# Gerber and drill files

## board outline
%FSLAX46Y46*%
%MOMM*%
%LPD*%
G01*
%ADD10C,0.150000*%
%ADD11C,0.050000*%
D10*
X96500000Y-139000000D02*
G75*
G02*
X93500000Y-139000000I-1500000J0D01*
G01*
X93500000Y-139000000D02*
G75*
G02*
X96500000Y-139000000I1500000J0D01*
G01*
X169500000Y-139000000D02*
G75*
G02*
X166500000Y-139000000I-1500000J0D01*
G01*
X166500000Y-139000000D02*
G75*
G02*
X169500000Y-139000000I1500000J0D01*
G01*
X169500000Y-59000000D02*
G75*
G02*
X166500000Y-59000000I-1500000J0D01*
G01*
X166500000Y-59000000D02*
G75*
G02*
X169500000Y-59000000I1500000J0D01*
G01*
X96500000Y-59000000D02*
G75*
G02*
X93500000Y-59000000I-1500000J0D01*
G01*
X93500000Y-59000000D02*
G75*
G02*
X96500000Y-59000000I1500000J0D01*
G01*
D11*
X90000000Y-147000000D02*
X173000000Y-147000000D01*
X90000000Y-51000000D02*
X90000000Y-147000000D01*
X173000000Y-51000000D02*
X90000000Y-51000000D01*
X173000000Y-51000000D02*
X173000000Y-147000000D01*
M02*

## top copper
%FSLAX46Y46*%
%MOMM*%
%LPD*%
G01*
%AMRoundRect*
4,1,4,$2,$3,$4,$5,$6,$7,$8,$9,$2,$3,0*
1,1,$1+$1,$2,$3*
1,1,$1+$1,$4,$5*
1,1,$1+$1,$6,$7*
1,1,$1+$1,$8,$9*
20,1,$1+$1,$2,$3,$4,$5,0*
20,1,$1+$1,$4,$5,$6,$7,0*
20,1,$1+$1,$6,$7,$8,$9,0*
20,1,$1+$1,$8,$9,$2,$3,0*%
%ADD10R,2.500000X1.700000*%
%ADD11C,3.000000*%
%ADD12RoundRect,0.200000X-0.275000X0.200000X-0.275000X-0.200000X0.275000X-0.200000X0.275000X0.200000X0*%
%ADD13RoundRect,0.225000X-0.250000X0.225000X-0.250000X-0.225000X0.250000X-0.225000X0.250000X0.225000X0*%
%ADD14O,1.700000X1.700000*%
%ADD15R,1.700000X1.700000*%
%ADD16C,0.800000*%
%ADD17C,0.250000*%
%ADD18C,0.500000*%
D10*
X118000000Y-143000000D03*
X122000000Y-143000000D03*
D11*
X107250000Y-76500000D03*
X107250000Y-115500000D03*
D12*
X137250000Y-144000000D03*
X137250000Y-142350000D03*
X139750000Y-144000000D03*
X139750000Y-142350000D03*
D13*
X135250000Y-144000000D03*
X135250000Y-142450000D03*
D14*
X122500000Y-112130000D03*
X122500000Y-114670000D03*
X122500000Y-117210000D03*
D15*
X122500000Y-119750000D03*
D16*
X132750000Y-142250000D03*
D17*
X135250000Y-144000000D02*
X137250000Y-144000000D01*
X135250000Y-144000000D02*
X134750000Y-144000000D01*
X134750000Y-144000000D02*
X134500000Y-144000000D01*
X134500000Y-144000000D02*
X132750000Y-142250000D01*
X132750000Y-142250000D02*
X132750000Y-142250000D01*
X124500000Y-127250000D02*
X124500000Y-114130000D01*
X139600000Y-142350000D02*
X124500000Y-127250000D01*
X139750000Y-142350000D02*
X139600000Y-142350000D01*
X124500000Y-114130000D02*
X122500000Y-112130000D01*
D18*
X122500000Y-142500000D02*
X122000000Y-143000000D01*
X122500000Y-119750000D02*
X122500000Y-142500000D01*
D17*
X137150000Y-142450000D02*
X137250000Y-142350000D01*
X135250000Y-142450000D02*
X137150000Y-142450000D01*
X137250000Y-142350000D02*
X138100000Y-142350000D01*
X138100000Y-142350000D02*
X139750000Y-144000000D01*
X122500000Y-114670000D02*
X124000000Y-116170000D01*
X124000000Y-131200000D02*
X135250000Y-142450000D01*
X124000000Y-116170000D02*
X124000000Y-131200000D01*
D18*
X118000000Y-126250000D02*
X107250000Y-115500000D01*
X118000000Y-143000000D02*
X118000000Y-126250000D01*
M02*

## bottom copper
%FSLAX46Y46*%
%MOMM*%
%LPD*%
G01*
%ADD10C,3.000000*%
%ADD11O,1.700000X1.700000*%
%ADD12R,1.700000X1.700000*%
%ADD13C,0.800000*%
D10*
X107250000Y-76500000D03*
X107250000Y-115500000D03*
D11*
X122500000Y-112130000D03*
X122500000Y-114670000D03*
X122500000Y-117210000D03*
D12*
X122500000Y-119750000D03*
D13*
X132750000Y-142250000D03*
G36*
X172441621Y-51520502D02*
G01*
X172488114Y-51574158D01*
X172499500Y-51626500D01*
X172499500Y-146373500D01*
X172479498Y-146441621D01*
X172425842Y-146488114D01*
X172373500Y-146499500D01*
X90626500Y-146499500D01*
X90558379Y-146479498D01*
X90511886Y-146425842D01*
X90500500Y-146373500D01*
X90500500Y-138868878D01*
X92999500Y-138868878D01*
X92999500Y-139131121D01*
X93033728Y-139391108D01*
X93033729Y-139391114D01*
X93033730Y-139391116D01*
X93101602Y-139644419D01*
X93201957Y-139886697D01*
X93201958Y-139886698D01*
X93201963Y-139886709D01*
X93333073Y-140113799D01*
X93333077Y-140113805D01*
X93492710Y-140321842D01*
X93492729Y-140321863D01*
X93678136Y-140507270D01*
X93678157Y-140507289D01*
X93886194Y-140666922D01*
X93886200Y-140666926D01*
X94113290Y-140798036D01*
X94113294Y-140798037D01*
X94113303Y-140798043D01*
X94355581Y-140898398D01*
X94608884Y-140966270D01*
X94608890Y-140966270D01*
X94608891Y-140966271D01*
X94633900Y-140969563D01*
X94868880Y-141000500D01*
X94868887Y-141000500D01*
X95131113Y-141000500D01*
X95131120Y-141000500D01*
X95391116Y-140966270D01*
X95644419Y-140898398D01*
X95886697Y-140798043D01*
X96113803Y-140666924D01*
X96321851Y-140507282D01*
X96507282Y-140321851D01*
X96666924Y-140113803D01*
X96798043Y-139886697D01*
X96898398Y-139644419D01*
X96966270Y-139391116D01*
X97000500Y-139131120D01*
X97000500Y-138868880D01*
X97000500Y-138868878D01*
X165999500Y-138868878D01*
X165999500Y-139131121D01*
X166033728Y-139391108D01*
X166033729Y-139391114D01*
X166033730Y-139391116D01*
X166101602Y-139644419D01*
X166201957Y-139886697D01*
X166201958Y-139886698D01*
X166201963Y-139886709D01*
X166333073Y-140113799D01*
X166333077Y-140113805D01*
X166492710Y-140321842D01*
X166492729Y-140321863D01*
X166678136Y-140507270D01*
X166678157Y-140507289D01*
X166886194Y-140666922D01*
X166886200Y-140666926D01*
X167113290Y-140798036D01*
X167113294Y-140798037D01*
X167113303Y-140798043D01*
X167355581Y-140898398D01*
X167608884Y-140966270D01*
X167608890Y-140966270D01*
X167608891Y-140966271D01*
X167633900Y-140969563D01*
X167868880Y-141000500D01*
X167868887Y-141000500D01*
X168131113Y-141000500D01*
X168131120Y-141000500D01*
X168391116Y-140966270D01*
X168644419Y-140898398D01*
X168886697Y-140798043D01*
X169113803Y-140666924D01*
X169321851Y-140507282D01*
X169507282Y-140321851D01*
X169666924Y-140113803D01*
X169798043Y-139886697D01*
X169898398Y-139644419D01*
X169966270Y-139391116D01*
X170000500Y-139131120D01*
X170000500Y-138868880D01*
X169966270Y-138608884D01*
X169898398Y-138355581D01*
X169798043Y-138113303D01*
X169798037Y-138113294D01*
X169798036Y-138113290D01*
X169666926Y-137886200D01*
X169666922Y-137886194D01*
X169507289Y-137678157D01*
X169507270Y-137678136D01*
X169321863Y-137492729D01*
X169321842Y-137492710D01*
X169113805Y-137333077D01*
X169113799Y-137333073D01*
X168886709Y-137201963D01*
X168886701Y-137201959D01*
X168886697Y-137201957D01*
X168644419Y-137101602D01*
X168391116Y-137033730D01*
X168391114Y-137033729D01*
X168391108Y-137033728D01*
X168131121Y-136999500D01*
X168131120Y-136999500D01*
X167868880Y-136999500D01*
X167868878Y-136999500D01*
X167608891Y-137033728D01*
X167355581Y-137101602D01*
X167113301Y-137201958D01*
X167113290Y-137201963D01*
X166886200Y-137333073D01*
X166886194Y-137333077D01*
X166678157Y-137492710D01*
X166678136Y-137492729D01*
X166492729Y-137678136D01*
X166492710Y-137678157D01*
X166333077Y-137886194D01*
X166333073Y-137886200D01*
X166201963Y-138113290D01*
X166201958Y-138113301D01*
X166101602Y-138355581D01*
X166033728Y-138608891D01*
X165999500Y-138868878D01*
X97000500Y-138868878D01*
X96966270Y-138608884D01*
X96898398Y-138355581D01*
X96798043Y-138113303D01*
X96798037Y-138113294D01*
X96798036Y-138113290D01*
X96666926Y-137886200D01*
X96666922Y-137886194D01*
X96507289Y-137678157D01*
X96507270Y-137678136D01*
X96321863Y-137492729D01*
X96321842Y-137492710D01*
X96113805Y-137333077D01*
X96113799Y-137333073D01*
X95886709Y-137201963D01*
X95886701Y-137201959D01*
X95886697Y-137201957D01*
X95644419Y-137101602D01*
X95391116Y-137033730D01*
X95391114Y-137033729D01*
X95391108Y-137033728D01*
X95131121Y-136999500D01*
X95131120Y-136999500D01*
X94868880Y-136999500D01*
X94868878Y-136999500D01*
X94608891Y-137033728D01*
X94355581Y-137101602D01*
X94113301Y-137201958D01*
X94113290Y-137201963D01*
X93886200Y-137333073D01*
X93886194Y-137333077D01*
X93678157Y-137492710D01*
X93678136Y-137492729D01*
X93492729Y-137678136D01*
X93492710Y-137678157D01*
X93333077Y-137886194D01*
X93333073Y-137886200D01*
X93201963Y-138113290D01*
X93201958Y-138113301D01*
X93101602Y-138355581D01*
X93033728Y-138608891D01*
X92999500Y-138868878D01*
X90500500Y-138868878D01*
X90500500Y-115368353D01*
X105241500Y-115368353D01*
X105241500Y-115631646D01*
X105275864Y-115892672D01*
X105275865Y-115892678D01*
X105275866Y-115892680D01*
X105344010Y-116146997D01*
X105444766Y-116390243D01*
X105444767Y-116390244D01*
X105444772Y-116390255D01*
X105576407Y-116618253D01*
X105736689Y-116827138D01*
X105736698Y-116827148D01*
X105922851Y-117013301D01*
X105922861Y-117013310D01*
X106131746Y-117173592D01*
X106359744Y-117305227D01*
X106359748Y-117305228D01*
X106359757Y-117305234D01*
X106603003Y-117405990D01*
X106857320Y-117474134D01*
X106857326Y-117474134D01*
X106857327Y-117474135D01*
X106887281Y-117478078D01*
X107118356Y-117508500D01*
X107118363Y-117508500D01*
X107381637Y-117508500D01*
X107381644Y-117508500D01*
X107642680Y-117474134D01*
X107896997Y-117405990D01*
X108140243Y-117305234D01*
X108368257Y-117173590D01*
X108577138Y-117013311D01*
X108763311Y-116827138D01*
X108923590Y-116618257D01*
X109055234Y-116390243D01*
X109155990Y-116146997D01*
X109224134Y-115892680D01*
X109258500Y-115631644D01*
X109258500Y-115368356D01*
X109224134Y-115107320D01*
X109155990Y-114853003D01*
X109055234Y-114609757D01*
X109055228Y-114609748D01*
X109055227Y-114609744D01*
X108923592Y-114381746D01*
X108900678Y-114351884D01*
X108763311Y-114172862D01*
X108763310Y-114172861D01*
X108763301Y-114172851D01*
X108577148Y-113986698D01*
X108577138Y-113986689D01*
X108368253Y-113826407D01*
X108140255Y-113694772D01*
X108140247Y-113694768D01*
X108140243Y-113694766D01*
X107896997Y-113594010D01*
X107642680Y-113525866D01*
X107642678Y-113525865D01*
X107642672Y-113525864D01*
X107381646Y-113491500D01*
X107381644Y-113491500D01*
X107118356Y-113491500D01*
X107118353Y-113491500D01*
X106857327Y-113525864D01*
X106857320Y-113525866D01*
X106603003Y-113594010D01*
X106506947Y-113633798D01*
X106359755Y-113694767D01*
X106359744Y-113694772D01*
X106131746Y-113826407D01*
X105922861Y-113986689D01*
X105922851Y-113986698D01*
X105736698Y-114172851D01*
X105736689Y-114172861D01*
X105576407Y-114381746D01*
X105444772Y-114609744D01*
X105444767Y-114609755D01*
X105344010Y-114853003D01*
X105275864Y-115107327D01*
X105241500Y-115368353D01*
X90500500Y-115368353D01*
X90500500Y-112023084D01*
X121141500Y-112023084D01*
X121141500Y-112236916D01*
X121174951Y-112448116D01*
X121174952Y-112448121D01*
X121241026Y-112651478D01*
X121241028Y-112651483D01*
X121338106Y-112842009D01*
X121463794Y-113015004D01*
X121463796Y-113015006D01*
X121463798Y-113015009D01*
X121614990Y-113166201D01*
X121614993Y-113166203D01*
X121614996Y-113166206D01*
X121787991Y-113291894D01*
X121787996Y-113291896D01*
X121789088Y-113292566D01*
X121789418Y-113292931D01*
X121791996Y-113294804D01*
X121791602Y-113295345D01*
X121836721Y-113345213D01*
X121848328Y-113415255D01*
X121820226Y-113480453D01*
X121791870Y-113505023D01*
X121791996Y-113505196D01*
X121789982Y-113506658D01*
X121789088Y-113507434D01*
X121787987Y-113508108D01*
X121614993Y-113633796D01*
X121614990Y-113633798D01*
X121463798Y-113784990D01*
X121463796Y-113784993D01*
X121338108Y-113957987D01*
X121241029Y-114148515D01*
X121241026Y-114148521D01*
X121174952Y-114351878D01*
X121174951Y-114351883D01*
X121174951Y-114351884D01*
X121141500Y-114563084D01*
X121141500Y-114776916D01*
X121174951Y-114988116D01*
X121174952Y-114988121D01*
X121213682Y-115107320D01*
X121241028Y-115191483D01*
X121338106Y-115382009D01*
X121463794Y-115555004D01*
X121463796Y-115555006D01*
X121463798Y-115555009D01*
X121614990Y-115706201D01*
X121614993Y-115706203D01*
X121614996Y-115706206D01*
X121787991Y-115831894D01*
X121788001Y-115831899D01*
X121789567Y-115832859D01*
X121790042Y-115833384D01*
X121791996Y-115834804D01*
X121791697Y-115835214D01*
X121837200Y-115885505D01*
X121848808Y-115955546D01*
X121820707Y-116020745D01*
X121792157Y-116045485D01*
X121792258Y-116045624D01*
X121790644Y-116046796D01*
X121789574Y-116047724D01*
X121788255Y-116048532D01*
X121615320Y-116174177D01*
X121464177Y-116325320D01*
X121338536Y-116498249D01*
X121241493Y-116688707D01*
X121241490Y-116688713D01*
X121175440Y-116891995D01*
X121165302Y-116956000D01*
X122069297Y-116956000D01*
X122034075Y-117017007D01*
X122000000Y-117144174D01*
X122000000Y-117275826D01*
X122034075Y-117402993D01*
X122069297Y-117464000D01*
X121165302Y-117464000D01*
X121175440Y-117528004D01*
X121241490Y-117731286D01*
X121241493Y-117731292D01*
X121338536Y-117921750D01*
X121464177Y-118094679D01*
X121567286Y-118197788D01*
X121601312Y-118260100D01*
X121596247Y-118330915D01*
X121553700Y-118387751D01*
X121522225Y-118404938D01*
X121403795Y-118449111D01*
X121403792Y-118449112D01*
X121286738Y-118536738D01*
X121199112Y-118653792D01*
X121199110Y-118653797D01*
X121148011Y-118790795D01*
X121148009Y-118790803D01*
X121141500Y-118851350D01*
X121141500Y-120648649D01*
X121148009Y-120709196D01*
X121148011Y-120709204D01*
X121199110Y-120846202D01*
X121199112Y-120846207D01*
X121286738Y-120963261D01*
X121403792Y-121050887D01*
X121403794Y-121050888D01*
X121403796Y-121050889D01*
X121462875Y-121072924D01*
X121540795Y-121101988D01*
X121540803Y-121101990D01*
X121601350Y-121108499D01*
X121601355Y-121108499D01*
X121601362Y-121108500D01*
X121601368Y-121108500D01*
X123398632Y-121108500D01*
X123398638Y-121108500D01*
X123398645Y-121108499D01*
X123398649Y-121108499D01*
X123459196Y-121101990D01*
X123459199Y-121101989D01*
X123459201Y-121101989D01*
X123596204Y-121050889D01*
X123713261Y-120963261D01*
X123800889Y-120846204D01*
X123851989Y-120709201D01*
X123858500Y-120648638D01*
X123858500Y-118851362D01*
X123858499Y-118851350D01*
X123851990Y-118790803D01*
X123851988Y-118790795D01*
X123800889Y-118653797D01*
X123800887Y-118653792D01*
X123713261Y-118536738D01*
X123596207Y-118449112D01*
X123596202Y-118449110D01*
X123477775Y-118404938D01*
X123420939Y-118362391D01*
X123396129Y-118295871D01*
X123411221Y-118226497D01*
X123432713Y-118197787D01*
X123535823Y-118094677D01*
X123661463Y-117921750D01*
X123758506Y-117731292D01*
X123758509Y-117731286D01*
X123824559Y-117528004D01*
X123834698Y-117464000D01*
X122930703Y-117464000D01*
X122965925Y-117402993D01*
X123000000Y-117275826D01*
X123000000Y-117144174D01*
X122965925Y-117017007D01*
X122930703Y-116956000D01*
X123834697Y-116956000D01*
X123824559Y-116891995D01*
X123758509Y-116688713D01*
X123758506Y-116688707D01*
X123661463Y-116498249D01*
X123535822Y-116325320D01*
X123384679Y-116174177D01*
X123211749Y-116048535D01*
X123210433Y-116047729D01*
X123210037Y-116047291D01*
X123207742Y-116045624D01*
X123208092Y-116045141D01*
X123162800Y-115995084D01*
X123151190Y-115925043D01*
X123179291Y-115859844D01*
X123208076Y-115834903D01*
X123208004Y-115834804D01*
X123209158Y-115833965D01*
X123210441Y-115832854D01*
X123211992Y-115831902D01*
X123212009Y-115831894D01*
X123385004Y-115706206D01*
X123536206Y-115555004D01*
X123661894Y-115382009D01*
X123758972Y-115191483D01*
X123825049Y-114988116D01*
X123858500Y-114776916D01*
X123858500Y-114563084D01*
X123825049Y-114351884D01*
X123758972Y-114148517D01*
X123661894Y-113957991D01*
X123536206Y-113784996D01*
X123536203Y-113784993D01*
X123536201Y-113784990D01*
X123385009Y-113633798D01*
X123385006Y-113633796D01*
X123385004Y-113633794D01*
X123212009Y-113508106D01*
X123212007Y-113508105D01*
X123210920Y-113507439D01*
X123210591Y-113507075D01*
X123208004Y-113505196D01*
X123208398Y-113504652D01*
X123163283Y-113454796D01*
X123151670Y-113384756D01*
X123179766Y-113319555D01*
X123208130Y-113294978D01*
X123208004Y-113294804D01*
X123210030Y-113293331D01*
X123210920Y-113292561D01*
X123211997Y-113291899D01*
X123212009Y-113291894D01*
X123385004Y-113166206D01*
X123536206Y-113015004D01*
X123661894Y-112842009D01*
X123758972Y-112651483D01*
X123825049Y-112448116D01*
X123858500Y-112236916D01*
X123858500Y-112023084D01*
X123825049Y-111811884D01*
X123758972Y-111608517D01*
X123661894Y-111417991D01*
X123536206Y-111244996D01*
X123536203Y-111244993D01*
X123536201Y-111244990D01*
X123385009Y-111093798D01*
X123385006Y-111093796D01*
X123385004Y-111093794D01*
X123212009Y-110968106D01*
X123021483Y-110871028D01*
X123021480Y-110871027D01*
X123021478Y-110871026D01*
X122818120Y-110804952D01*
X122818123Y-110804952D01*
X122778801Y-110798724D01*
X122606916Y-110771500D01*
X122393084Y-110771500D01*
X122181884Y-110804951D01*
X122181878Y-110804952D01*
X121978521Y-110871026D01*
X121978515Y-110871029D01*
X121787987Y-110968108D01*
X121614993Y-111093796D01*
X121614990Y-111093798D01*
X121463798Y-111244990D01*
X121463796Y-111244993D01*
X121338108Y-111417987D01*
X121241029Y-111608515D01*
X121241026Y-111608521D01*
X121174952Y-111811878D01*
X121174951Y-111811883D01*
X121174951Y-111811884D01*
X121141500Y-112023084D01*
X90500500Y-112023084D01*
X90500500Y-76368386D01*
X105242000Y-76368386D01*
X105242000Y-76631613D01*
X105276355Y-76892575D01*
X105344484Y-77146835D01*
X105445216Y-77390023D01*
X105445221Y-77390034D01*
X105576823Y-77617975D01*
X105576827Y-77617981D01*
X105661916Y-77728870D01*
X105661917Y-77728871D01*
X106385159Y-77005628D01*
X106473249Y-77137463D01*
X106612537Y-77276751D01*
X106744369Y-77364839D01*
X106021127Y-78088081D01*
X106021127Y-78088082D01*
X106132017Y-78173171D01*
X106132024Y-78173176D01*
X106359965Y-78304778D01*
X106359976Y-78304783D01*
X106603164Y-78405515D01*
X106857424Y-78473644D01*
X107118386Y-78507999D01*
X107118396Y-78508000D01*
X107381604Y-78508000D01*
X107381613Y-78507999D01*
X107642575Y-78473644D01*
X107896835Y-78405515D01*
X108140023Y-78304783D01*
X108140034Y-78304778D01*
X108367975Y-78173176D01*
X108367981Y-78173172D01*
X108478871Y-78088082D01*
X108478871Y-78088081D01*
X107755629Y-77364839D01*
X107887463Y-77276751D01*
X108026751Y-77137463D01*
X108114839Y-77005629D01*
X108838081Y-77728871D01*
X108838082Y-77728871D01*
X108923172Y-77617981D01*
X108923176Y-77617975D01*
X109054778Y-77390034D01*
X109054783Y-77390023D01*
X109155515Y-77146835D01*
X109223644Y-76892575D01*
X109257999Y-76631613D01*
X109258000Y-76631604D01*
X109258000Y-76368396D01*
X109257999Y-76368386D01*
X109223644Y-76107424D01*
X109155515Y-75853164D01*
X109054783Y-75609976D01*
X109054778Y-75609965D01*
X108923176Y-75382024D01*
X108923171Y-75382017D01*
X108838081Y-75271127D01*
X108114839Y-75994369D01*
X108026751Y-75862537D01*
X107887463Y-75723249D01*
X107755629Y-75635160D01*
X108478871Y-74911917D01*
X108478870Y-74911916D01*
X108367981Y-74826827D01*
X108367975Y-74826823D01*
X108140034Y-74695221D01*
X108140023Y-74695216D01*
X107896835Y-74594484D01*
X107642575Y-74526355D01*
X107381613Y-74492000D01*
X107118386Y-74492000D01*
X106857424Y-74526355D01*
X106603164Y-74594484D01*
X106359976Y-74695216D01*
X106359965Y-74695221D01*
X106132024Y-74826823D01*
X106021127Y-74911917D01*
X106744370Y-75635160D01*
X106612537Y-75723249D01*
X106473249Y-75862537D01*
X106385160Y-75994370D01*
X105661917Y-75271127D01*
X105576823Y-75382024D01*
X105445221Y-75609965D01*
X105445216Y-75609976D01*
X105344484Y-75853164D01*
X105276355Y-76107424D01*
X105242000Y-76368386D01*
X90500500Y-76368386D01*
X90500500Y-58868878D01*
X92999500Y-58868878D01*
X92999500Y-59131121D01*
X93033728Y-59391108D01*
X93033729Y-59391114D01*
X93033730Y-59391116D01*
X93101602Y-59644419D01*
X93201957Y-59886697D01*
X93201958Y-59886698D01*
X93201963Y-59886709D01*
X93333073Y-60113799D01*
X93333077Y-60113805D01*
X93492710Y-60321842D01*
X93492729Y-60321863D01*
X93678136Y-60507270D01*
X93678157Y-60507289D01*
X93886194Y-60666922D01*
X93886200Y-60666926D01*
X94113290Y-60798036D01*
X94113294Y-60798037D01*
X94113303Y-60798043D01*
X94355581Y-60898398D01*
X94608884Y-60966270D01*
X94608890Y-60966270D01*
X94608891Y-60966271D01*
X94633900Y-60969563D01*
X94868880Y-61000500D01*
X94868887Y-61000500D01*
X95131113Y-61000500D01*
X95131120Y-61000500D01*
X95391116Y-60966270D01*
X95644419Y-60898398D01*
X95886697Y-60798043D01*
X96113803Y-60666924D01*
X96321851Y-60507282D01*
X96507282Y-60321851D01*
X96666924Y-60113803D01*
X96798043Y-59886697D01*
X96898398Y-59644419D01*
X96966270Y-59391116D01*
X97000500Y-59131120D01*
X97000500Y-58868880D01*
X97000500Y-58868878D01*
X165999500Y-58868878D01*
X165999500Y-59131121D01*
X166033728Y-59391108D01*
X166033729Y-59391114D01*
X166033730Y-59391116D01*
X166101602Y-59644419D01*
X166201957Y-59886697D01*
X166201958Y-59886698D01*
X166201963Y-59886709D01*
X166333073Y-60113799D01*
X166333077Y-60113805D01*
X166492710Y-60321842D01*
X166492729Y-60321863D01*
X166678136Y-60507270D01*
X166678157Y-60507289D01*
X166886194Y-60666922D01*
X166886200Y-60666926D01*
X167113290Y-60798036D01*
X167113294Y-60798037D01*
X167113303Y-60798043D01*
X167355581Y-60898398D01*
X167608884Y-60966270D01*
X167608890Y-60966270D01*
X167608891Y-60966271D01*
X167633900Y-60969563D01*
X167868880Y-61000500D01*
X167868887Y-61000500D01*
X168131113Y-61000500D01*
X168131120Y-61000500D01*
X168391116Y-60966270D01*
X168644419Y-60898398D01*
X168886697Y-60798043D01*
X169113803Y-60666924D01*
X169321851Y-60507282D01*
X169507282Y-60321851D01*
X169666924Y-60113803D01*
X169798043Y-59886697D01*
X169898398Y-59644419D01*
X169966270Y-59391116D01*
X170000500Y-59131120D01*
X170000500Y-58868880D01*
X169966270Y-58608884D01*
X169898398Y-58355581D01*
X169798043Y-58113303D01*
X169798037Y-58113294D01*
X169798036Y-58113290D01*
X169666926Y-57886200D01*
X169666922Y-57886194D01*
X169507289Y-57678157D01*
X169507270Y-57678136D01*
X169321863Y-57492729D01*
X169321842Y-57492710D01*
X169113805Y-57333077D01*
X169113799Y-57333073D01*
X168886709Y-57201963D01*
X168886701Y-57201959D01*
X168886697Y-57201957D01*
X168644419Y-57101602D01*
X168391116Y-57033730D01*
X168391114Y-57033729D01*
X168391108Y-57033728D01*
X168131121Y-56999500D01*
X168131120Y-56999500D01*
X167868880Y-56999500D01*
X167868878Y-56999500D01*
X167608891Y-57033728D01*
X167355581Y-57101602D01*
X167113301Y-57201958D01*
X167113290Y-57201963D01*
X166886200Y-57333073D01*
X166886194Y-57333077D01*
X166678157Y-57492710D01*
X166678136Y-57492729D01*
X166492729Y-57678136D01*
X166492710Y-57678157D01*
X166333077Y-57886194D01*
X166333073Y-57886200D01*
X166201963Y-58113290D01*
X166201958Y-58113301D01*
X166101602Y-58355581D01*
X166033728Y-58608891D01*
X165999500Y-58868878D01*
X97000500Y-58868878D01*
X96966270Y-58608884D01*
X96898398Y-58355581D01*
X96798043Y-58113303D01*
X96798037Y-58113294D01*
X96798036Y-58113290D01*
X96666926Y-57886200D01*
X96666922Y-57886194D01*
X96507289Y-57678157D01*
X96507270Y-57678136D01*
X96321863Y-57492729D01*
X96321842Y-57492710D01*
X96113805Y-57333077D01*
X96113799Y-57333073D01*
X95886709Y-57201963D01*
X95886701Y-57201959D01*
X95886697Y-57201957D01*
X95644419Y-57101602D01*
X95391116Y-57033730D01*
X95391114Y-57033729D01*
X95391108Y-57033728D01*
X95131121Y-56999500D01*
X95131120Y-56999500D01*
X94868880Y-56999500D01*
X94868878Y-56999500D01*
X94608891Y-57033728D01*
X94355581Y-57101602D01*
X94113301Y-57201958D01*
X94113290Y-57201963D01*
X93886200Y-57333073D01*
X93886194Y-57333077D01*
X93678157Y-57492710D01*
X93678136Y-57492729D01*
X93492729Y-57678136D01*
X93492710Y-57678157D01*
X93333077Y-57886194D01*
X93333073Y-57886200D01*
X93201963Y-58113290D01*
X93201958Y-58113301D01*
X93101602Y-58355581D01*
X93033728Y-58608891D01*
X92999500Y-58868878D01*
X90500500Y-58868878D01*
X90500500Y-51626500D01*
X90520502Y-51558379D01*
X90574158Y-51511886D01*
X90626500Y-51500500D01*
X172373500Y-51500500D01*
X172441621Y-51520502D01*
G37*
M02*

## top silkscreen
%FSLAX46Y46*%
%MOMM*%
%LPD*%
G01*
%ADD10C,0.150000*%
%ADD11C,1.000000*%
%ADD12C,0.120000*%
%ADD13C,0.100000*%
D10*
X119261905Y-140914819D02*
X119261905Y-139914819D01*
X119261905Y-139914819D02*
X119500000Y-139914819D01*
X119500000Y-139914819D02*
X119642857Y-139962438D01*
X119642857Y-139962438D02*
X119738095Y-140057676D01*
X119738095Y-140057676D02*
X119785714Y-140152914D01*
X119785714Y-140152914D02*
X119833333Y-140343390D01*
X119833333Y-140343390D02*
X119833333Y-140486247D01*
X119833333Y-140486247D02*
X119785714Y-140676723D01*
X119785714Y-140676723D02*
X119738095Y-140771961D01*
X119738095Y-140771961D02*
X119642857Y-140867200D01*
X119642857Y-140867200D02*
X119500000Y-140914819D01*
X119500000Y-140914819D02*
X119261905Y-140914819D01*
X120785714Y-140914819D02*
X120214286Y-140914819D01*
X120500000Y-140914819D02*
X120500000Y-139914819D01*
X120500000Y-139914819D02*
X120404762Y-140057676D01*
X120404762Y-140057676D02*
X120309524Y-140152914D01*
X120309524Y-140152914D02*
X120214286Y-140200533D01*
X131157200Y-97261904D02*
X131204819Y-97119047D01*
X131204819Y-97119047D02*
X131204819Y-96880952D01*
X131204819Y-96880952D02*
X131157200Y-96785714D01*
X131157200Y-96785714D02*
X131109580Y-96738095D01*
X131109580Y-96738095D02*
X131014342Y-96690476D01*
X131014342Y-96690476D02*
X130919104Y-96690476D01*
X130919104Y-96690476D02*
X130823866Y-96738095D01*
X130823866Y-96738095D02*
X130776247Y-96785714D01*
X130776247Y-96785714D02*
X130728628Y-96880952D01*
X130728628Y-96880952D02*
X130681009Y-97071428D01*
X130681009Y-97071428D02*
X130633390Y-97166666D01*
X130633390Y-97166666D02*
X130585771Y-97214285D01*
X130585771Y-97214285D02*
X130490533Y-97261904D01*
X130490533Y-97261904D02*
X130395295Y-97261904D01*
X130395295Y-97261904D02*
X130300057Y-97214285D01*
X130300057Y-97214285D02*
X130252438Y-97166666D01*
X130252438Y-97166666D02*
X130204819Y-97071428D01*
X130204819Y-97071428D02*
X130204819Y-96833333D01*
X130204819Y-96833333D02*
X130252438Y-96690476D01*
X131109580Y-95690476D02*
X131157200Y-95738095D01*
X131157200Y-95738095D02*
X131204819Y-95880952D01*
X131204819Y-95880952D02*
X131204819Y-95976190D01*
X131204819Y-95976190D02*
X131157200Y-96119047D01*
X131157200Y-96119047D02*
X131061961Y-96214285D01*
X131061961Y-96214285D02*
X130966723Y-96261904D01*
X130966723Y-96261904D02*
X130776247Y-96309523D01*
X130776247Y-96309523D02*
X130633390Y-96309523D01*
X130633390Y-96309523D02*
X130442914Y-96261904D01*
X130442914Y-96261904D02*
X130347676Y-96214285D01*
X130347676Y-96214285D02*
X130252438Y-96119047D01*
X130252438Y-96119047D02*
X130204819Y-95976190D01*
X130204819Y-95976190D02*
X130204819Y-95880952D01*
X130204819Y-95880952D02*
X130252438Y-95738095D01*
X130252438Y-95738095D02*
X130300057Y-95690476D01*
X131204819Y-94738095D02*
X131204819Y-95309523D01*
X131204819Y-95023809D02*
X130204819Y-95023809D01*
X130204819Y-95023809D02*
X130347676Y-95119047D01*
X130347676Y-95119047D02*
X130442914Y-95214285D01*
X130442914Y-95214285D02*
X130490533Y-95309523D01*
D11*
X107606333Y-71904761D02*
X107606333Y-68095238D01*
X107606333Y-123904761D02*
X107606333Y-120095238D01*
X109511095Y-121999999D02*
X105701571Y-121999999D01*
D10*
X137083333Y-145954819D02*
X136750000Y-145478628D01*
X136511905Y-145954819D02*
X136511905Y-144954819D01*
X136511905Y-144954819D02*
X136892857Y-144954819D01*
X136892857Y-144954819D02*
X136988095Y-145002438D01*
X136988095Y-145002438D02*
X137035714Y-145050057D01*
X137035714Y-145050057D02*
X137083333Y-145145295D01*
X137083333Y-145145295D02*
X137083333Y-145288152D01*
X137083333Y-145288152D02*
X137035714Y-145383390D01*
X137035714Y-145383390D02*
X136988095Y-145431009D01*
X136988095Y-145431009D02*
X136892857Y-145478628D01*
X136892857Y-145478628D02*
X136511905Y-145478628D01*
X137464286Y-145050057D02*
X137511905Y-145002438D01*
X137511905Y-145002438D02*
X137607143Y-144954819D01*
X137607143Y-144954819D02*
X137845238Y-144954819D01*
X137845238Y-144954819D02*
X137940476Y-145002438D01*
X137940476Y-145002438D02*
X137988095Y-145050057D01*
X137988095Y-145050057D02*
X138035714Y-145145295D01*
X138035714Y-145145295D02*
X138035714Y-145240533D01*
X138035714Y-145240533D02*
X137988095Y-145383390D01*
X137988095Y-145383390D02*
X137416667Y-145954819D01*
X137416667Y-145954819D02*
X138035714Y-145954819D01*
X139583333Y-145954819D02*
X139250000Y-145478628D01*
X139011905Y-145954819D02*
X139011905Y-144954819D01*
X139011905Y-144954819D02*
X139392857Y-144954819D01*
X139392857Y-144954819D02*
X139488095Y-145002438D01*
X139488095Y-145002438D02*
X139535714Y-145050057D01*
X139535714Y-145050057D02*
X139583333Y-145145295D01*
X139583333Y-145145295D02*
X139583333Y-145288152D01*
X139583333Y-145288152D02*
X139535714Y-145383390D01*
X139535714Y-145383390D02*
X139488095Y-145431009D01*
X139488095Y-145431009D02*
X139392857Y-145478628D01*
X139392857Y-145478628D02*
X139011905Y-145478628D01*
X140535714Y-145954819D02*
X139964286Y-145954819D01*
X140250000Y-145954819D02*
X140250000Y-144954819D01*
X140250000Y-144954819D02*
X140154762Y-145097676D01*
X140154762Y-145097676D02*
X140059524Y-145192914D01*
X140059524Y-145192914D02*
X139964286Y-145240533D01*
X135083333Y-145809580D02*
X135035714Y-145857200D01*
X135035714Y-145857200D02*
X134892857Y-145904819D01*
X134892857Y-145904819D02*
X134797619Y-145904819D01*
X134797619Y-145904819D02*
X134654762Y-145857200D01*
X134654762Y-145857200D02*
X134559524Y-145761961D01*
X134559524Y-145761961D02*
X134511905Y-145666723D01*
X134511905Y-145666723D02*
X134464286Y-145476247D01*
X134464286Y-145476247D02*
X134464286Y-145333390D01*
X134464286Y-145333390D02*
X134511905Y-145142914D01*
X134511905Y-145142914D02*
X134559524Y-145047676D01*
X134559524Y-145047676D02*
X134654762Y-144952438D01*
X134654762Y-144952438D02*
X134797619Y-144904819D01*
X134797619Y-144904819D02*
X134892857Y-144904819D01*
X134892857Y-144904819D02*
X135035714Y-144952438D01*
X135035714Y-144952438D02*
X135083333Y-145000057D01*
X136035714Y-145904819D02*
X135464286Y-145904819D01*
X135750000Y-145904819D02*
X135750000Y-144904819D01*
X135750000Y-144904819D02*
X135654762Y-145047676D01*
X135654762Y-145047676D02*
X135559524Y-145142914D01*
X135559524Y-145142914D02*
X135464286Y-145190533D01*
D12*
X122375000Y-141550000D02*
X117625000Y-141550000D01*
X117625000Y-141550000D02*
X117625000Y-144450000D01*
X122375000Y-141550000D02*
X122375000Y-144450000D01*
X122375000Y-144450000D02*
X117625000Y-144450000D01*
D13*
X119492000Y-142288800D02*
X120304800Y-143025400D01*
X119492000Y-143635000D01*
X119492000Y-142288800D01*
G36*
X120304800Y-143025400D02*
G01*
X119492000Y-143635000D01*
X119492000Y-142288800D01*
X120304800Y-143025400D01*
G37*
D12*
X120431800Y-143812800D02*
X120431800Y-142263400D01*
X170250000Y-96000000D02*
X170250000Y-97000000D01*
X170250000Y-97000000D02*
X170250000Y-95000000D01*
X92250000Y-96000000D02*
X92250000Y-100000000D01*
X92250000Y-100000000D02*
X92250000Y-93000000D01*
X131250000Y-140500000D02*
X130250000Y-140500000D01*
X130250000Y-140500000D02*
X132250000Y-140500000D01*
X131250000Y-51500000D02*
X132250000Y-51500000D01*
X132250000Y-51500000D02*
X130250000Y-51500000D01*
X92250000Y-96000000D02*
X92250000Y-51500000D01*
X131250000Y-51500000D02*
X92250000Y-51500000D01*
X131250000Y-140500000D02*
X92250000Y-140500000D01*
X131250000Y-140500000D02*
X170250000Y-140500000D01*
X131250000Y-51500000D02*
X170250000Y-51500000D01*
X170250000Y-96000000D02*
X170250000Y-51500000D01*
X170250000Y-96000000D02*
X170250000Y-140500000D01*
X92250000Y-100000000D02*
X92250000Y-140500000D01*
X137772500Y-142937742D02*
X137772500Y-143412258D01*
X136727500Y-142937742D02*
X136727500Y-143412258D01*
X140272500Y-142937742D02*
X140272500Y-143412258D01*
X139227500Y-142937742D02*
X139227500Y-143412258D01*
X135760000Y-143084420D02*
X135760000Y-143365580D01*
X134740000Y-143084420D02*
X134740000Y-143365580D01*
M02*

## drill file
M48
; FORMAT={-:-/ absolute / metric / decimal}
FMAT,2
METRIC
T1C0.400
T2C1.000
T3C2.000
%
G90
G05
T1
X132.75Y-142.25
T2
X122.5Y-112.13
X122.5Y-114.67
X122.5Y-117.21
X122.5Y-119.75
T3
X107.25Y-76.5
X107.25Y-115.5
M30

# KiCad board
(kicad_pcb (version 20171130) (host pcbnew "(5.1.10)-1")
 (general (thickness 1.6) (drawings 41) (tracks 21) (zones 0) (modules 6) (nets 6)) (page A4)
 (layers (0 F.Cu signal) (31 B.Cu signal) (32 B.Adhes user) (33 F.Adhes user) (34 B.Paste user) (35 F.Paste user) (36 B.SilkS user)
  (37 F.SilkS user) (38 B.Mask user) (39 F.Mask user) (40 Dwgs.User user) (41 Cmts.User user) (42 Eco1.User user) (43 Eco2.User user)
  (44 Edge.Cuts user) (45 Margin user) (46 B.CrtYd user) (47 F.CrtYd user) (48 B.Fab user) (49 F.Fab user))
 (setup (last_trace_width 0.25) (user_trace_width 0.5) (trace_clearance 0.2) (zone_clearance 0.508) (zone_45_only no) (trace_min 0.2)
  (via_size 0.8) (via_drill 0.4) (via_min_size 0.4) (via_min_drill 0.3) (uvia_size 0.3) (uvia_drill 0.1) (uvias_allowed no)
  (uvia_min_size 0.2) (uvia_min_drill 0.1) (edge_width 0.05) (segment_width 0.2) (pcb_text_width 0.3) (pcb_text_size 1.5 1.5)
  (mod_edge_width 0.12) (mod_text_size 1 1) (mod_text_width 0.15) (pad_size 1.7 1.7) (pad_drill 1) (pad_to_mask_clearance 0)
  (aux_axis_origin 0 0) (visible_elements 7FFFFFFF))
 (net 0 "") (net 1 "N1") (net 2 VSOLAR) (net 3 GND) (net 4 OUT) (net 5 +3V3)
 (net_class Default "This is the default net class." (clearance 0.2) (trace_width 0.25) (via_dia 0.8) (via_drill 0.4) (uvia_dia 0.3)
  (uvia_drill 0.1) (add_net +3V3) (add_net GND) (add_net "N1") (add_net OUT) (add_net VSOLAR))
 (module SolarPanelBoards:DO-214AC (layer F.Cu) (at 120 143 180)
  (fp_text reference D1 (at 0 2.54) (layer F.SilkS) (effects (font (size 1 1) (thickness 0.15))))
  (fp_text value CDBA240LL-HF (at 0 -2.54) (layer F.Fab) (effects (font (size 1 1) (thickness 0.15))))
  (fp_line (start -2.375 1.45) (end 2.375 1.45) (layer F.SilkS) (width 0.12))
  (fp_line (start 2.375 1.45) (end 2.375 -1.45) (layer F.SilkS) (width 0.12))
  (fp_line (start -2.375 1.45) (end -2.375 -1.45) (layer F.SilkS) (width 0.12))
  (fp_line (start -2.375 -1.45) (end 2.375 -1.45) (layer F.SilkS) (width 0.12))
  (fp_poly (pts (xy 0.508 0.7112) (xy -0.3048 -0.0254) (xy 0.508 -0.635)) (layer F.SilkS) (width 0.1))
  (fp_line (start -0.4318 -0.8128) (end -0.4318 0.7366) (layer F.SilkS) (width 0.12))
  (pad 2 smd rect (at 2 0 180) (size 2.5 1.7) (layers F.Cu F.Paste F.Mask) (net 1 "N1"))
  (pad 1 smd rect (at -2 0 180) (size 2.5 1.7) (layers F.Cu F.Paste F.Mask) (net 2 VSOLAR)))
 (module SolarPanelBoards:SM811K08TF (layer F.Cu) (at 131.25 96 270)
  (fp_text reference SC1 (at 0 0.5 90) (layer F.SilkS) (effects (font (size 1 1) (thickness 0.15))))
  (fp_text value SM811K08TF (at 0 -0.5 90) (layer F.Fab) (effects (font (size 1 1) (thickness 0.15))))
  (fp_line (start 0 -39) (end 1 -39) (layer F.SilkS) (width 0.12))
  (fp_line (start 1 -39) (end -1 -39) (layer F.SilkS) (width 0.12))
  (fp_line (start 0 39) (end 4 39) (layer F.SilkS) (width 0.12))
  (fp_line (start 4 39) (end -3 39) (layer F.SilkS) (width 0.12))
  (fp_line (start 44.5 0) (end 44.5 1) (layer F.SilkS) (width 0.12))
  (fp_line (start 44.5 1) (end 44.5 -1) (layer F.SilkS) (width 0.12))
  (fp_line (start -44.5 0) (end -44.5 -1) (layer F.SilkS) (width 0.12))
  (fp_line (start -44.5 -1) (end -44.5 1) (layer F.SilkS) (width 0.12))
  (fp_line (start 0 39) (end -44.5 39) (layer F.SilkS) (width 0.12))
  (fp_line (start -44.5 0) (end -44.5 39) (layer F.SilkS) (width 0.12))
  (fp_line (start 44.5 0) (end 44.5 39) (layer F.SilkS) (width 0.12))
  (fp_line (start 44.5 0) (end 44.5 -39) (layer F.SilkS) (width 0.12))
  (fp_line (start -44.5 0) (end -44.5 -39) (layer F.SilkS) (width 0.12))
  (fp_line (start 0 -39) (end -44.5 -39) (layer F.SilkS) (width 0.12))
  (fp_line (start 0 -39) (end 44.5 -39) (layer F.SilkS) (width 0.12))
  (fp_line (start 4 39) (end 44.5 39) (layer F.SilkS) (width 0.12))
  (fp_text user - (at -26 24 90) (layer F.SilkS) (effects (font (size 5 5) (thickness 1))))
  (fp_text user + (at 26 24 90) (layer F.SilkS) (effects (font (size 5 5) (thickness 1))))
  (pad 2 thru_hole circle (at -19.5 24 270) (size 3 3) (drill 2) (layers *.Cu *.Mask) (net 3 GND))
  (pad 1 thru_hole circle (at 19.5 24 270) (size 3 3) (drill 2) (layers *.Cu *.Mask) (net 1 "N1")))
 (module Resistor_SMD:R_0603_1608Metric (layer F.Cu) (at 137.25 143.175 270)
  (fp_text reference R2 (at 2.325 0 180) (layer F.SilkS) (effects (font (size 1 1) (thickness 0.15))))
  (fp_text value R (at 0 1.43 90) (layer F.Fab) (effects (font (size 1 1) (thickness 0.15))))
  (fp_line (start -0.237258 -0.5225) (end 0.237258 -0.5225) (layer F.SilkS) (width 0.12))
  (fp_line (start -0.237258 0.5225) (end 0.237258 0.5225) (layer F.SilkS) (width 0.12))
  (pad 2 smd roundrect (at 0.825 0 270) (size 0.8 0.95) (layers F.Cu F.Paste F.Mask) (roundrect_rratio 0.25) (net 3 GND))
  (pad 1 smd roundrect (at -0.825 0 270) (size 0.8 0.95) (layers F.Cu F.Paste F.Mask) (roundrect_rratio 0.25) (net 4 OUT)))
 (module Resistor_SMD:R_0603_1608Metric (layer F.Cu) (at 139.75 143.175 270)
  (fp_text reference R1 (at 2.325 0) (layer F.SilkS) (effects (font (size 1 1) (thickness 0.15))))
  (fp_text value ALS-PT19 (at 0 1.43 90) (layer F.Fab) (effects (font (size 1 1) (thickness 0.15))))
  (fp_line (start -0.237258 -0.5225) (end 0.237258 -0.5225) (layer F.SilkS) (width 0.12))
  (fp_line (start -0.237258 0.5225) (end 0.237258 0.5225) (layer F.SilkS) (width 0.12))
  (pad 2 smd roundrect (at 0.825 0 270) (size 0.8 0.95) (layers F.Cu F.Paste F.Mask) (roundrect_rratio 0.25) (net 4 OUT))
  (pad 1 smd roundrect (at -0.825 0 270) (size 0.8 0.95) (layers F.Cu F.Paste F.Mask) (roundrect_rratio 0.25) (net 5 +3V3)))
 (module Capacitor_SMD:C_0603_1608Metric (layer F.Cu) (at 135.25 143.225 270)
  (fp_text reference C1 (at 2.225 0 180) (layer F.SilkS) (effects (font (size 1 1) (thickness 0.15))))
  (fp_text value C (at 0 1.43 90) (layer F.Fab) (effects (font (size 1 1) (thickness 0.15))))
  (fp_line (start -0.14058 -0.51) (end 0.14058 -0.51) (layer F.SilkS) (width 0.12))
  (fp_line (start -0.14058 0.51) (end 0.14058 0.51) (layer F.SilkS) (width 0.12))
  (pad 2 smd roundrect (at 0.775 0 270) (size 0.9 0.95) (layers F.Cu F.Paste F.Mask) (roundrect_rratio 0.25) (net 3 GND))
  (pad 1 smd roundrect (at -0.775 0 270) (size 0.9 0.95) (layers F.Cu F.Paste F.Mask) (roundrect_rratio 0.25) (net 4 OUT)))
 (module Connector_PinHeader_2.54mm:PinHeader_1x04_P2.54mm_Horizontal (layer B.Cu) (at 122.5 119.75)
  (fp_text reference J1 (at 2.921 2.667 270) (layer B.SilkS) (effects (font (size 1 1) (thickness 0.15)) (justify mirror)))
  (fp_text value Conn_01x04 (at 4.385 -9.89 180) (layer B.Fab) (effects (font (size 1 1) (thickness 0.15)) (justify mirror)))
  (pad 4 thru_hole oval (at 0 -7.62) (size 1.7 1.7) (drill 1) (layers *.Cu *.Mask) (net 5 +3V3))
  (pad 3 thru_hole oval (at 0 -5.08) (size 1.7 1.7) (drill 1) (layers *.Cu *.Mask) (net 4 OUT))
  (pad 2 thru_hole oval (at 0 -2.54) (size 1.7 1.7) (drill 1) (layers *.Cu *.Mask) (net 3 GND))
  (pad 1 thru_hole rect (at 0 0) (size 1.7 1.7) (drill 1) (layers *.Cu *.Mask) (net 2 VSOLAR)))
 (gr_circle (center 95 139) (end 96.5 139) (layer Edge.Cuts) (width 0.15))
 (gr_circle (center 168 139) (end 169.5 139) (layer Edge.Cuts) (width 0.15))
 (gr_circle (center 168 59) (end 169.5 59) (layer Edge.Cuts) (width 0.15))
 (gr_circle (center 95 59) (end 96.5 59) (layer Edge.Cuts) (width 0.15))
 (gr_line (start 90 147) (end 173 147) (layer Edge.Cuts) (width 0.05))
 (gr_line (start 90 51) (end 90 147) (layer Edge.Cuts) (width 0.05))
 (gr_line (start 173 51) (end 90 51) (layer Edge.Cuts) (width 0.05))
 (gr_line (start 173 51) (end 173 147) (layer Edge.Cuts) (width 0.05))
 (segment (start 135.25 144) (end 137.25 144) (width 0.25) (layer F.Cu) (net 3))
 (segment (start 135.25 144) (end 134.75 144) (width 0.25) (layer F.Cu) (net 3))
 (segment (start 134.75 144) (end 134.5 144) (width 0.25) (layer F.Cu) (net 3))
 (segment (start 134.5 144) (end 132.75 142.25) (width 0.25) (layer F.Cu) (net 3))
 (segment (start 132.75 142.25) (end 132.75 142.25) (width 0.25) (layer F.Cu) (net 3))
 (via (at 132.75 142.25) (size 0.8) (drill 0.4) (layers F.Cu B.Cu) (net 3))
 (segment (start 124.5 127.25) (end 124.5 114.13) (width 0.25) (layer F.Cu) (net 5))
 (segment (start 139.6 142.35) (end 124.5 127.25) (width 0.25) (layer F.Cu) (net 5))
 (segment (start 139.75 142.35) (end 139.6 142.35) (width 0.25) (layer F.Cu) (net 5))
 (segment (start 124.5 114.13) (end 122.5 112.13) (width 0.25) (layer F.Cu) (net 5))
 (segment (start 122.5 142.5) (end 122 143) (width 0.5) (layer F.Cu) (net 2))
 (segment (start 122.5 119.75) (end 122.5 142.5) (width 0.5) (layer F.Cu) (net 2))
 (segment (start 137.15 142.45) (end 137.25 142.35) (width 0.25) (layer F.Cu) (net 4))
 (segment (start 135.25 142.45) (end 137.15 142.45) (width 0.25) (layer F.Cu) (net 4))
 (segment (start 137.25 142.35) (end 138.1 142.35) (width 0.25) (layer F.Cu) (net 4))
 (segment (start 138.1 142.35) (end 139.75 144) (width 0.25) (layer F.Cu) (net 4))
 (segment (start 122.5 114.67) (end 124 116.17) (width 0.25) (layer F.Cu) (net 4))
 (segment (start 124 131.2) (end 135.25 142.45) (width 0.25) (layer F.Cu) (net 4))
 (segment (start 124 116.17) (end 124 131.2) (width 0.25) (layer F.Cu) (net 4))
 (segment (start 118 126.25) (end 107.25 115.5) (width 0.5) (layer F.Cu) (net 1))
 (segment (start 118 143) (end 118 126.25) (width 0.5) (layer F.Cu) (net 1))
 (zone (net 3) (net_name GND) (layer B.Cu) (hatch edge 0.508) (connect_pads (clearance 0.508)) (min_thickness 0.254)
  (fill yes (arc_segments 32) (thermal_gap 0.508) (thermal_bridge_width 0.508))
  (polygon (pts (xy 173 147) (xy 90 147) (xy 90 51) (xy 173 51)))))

